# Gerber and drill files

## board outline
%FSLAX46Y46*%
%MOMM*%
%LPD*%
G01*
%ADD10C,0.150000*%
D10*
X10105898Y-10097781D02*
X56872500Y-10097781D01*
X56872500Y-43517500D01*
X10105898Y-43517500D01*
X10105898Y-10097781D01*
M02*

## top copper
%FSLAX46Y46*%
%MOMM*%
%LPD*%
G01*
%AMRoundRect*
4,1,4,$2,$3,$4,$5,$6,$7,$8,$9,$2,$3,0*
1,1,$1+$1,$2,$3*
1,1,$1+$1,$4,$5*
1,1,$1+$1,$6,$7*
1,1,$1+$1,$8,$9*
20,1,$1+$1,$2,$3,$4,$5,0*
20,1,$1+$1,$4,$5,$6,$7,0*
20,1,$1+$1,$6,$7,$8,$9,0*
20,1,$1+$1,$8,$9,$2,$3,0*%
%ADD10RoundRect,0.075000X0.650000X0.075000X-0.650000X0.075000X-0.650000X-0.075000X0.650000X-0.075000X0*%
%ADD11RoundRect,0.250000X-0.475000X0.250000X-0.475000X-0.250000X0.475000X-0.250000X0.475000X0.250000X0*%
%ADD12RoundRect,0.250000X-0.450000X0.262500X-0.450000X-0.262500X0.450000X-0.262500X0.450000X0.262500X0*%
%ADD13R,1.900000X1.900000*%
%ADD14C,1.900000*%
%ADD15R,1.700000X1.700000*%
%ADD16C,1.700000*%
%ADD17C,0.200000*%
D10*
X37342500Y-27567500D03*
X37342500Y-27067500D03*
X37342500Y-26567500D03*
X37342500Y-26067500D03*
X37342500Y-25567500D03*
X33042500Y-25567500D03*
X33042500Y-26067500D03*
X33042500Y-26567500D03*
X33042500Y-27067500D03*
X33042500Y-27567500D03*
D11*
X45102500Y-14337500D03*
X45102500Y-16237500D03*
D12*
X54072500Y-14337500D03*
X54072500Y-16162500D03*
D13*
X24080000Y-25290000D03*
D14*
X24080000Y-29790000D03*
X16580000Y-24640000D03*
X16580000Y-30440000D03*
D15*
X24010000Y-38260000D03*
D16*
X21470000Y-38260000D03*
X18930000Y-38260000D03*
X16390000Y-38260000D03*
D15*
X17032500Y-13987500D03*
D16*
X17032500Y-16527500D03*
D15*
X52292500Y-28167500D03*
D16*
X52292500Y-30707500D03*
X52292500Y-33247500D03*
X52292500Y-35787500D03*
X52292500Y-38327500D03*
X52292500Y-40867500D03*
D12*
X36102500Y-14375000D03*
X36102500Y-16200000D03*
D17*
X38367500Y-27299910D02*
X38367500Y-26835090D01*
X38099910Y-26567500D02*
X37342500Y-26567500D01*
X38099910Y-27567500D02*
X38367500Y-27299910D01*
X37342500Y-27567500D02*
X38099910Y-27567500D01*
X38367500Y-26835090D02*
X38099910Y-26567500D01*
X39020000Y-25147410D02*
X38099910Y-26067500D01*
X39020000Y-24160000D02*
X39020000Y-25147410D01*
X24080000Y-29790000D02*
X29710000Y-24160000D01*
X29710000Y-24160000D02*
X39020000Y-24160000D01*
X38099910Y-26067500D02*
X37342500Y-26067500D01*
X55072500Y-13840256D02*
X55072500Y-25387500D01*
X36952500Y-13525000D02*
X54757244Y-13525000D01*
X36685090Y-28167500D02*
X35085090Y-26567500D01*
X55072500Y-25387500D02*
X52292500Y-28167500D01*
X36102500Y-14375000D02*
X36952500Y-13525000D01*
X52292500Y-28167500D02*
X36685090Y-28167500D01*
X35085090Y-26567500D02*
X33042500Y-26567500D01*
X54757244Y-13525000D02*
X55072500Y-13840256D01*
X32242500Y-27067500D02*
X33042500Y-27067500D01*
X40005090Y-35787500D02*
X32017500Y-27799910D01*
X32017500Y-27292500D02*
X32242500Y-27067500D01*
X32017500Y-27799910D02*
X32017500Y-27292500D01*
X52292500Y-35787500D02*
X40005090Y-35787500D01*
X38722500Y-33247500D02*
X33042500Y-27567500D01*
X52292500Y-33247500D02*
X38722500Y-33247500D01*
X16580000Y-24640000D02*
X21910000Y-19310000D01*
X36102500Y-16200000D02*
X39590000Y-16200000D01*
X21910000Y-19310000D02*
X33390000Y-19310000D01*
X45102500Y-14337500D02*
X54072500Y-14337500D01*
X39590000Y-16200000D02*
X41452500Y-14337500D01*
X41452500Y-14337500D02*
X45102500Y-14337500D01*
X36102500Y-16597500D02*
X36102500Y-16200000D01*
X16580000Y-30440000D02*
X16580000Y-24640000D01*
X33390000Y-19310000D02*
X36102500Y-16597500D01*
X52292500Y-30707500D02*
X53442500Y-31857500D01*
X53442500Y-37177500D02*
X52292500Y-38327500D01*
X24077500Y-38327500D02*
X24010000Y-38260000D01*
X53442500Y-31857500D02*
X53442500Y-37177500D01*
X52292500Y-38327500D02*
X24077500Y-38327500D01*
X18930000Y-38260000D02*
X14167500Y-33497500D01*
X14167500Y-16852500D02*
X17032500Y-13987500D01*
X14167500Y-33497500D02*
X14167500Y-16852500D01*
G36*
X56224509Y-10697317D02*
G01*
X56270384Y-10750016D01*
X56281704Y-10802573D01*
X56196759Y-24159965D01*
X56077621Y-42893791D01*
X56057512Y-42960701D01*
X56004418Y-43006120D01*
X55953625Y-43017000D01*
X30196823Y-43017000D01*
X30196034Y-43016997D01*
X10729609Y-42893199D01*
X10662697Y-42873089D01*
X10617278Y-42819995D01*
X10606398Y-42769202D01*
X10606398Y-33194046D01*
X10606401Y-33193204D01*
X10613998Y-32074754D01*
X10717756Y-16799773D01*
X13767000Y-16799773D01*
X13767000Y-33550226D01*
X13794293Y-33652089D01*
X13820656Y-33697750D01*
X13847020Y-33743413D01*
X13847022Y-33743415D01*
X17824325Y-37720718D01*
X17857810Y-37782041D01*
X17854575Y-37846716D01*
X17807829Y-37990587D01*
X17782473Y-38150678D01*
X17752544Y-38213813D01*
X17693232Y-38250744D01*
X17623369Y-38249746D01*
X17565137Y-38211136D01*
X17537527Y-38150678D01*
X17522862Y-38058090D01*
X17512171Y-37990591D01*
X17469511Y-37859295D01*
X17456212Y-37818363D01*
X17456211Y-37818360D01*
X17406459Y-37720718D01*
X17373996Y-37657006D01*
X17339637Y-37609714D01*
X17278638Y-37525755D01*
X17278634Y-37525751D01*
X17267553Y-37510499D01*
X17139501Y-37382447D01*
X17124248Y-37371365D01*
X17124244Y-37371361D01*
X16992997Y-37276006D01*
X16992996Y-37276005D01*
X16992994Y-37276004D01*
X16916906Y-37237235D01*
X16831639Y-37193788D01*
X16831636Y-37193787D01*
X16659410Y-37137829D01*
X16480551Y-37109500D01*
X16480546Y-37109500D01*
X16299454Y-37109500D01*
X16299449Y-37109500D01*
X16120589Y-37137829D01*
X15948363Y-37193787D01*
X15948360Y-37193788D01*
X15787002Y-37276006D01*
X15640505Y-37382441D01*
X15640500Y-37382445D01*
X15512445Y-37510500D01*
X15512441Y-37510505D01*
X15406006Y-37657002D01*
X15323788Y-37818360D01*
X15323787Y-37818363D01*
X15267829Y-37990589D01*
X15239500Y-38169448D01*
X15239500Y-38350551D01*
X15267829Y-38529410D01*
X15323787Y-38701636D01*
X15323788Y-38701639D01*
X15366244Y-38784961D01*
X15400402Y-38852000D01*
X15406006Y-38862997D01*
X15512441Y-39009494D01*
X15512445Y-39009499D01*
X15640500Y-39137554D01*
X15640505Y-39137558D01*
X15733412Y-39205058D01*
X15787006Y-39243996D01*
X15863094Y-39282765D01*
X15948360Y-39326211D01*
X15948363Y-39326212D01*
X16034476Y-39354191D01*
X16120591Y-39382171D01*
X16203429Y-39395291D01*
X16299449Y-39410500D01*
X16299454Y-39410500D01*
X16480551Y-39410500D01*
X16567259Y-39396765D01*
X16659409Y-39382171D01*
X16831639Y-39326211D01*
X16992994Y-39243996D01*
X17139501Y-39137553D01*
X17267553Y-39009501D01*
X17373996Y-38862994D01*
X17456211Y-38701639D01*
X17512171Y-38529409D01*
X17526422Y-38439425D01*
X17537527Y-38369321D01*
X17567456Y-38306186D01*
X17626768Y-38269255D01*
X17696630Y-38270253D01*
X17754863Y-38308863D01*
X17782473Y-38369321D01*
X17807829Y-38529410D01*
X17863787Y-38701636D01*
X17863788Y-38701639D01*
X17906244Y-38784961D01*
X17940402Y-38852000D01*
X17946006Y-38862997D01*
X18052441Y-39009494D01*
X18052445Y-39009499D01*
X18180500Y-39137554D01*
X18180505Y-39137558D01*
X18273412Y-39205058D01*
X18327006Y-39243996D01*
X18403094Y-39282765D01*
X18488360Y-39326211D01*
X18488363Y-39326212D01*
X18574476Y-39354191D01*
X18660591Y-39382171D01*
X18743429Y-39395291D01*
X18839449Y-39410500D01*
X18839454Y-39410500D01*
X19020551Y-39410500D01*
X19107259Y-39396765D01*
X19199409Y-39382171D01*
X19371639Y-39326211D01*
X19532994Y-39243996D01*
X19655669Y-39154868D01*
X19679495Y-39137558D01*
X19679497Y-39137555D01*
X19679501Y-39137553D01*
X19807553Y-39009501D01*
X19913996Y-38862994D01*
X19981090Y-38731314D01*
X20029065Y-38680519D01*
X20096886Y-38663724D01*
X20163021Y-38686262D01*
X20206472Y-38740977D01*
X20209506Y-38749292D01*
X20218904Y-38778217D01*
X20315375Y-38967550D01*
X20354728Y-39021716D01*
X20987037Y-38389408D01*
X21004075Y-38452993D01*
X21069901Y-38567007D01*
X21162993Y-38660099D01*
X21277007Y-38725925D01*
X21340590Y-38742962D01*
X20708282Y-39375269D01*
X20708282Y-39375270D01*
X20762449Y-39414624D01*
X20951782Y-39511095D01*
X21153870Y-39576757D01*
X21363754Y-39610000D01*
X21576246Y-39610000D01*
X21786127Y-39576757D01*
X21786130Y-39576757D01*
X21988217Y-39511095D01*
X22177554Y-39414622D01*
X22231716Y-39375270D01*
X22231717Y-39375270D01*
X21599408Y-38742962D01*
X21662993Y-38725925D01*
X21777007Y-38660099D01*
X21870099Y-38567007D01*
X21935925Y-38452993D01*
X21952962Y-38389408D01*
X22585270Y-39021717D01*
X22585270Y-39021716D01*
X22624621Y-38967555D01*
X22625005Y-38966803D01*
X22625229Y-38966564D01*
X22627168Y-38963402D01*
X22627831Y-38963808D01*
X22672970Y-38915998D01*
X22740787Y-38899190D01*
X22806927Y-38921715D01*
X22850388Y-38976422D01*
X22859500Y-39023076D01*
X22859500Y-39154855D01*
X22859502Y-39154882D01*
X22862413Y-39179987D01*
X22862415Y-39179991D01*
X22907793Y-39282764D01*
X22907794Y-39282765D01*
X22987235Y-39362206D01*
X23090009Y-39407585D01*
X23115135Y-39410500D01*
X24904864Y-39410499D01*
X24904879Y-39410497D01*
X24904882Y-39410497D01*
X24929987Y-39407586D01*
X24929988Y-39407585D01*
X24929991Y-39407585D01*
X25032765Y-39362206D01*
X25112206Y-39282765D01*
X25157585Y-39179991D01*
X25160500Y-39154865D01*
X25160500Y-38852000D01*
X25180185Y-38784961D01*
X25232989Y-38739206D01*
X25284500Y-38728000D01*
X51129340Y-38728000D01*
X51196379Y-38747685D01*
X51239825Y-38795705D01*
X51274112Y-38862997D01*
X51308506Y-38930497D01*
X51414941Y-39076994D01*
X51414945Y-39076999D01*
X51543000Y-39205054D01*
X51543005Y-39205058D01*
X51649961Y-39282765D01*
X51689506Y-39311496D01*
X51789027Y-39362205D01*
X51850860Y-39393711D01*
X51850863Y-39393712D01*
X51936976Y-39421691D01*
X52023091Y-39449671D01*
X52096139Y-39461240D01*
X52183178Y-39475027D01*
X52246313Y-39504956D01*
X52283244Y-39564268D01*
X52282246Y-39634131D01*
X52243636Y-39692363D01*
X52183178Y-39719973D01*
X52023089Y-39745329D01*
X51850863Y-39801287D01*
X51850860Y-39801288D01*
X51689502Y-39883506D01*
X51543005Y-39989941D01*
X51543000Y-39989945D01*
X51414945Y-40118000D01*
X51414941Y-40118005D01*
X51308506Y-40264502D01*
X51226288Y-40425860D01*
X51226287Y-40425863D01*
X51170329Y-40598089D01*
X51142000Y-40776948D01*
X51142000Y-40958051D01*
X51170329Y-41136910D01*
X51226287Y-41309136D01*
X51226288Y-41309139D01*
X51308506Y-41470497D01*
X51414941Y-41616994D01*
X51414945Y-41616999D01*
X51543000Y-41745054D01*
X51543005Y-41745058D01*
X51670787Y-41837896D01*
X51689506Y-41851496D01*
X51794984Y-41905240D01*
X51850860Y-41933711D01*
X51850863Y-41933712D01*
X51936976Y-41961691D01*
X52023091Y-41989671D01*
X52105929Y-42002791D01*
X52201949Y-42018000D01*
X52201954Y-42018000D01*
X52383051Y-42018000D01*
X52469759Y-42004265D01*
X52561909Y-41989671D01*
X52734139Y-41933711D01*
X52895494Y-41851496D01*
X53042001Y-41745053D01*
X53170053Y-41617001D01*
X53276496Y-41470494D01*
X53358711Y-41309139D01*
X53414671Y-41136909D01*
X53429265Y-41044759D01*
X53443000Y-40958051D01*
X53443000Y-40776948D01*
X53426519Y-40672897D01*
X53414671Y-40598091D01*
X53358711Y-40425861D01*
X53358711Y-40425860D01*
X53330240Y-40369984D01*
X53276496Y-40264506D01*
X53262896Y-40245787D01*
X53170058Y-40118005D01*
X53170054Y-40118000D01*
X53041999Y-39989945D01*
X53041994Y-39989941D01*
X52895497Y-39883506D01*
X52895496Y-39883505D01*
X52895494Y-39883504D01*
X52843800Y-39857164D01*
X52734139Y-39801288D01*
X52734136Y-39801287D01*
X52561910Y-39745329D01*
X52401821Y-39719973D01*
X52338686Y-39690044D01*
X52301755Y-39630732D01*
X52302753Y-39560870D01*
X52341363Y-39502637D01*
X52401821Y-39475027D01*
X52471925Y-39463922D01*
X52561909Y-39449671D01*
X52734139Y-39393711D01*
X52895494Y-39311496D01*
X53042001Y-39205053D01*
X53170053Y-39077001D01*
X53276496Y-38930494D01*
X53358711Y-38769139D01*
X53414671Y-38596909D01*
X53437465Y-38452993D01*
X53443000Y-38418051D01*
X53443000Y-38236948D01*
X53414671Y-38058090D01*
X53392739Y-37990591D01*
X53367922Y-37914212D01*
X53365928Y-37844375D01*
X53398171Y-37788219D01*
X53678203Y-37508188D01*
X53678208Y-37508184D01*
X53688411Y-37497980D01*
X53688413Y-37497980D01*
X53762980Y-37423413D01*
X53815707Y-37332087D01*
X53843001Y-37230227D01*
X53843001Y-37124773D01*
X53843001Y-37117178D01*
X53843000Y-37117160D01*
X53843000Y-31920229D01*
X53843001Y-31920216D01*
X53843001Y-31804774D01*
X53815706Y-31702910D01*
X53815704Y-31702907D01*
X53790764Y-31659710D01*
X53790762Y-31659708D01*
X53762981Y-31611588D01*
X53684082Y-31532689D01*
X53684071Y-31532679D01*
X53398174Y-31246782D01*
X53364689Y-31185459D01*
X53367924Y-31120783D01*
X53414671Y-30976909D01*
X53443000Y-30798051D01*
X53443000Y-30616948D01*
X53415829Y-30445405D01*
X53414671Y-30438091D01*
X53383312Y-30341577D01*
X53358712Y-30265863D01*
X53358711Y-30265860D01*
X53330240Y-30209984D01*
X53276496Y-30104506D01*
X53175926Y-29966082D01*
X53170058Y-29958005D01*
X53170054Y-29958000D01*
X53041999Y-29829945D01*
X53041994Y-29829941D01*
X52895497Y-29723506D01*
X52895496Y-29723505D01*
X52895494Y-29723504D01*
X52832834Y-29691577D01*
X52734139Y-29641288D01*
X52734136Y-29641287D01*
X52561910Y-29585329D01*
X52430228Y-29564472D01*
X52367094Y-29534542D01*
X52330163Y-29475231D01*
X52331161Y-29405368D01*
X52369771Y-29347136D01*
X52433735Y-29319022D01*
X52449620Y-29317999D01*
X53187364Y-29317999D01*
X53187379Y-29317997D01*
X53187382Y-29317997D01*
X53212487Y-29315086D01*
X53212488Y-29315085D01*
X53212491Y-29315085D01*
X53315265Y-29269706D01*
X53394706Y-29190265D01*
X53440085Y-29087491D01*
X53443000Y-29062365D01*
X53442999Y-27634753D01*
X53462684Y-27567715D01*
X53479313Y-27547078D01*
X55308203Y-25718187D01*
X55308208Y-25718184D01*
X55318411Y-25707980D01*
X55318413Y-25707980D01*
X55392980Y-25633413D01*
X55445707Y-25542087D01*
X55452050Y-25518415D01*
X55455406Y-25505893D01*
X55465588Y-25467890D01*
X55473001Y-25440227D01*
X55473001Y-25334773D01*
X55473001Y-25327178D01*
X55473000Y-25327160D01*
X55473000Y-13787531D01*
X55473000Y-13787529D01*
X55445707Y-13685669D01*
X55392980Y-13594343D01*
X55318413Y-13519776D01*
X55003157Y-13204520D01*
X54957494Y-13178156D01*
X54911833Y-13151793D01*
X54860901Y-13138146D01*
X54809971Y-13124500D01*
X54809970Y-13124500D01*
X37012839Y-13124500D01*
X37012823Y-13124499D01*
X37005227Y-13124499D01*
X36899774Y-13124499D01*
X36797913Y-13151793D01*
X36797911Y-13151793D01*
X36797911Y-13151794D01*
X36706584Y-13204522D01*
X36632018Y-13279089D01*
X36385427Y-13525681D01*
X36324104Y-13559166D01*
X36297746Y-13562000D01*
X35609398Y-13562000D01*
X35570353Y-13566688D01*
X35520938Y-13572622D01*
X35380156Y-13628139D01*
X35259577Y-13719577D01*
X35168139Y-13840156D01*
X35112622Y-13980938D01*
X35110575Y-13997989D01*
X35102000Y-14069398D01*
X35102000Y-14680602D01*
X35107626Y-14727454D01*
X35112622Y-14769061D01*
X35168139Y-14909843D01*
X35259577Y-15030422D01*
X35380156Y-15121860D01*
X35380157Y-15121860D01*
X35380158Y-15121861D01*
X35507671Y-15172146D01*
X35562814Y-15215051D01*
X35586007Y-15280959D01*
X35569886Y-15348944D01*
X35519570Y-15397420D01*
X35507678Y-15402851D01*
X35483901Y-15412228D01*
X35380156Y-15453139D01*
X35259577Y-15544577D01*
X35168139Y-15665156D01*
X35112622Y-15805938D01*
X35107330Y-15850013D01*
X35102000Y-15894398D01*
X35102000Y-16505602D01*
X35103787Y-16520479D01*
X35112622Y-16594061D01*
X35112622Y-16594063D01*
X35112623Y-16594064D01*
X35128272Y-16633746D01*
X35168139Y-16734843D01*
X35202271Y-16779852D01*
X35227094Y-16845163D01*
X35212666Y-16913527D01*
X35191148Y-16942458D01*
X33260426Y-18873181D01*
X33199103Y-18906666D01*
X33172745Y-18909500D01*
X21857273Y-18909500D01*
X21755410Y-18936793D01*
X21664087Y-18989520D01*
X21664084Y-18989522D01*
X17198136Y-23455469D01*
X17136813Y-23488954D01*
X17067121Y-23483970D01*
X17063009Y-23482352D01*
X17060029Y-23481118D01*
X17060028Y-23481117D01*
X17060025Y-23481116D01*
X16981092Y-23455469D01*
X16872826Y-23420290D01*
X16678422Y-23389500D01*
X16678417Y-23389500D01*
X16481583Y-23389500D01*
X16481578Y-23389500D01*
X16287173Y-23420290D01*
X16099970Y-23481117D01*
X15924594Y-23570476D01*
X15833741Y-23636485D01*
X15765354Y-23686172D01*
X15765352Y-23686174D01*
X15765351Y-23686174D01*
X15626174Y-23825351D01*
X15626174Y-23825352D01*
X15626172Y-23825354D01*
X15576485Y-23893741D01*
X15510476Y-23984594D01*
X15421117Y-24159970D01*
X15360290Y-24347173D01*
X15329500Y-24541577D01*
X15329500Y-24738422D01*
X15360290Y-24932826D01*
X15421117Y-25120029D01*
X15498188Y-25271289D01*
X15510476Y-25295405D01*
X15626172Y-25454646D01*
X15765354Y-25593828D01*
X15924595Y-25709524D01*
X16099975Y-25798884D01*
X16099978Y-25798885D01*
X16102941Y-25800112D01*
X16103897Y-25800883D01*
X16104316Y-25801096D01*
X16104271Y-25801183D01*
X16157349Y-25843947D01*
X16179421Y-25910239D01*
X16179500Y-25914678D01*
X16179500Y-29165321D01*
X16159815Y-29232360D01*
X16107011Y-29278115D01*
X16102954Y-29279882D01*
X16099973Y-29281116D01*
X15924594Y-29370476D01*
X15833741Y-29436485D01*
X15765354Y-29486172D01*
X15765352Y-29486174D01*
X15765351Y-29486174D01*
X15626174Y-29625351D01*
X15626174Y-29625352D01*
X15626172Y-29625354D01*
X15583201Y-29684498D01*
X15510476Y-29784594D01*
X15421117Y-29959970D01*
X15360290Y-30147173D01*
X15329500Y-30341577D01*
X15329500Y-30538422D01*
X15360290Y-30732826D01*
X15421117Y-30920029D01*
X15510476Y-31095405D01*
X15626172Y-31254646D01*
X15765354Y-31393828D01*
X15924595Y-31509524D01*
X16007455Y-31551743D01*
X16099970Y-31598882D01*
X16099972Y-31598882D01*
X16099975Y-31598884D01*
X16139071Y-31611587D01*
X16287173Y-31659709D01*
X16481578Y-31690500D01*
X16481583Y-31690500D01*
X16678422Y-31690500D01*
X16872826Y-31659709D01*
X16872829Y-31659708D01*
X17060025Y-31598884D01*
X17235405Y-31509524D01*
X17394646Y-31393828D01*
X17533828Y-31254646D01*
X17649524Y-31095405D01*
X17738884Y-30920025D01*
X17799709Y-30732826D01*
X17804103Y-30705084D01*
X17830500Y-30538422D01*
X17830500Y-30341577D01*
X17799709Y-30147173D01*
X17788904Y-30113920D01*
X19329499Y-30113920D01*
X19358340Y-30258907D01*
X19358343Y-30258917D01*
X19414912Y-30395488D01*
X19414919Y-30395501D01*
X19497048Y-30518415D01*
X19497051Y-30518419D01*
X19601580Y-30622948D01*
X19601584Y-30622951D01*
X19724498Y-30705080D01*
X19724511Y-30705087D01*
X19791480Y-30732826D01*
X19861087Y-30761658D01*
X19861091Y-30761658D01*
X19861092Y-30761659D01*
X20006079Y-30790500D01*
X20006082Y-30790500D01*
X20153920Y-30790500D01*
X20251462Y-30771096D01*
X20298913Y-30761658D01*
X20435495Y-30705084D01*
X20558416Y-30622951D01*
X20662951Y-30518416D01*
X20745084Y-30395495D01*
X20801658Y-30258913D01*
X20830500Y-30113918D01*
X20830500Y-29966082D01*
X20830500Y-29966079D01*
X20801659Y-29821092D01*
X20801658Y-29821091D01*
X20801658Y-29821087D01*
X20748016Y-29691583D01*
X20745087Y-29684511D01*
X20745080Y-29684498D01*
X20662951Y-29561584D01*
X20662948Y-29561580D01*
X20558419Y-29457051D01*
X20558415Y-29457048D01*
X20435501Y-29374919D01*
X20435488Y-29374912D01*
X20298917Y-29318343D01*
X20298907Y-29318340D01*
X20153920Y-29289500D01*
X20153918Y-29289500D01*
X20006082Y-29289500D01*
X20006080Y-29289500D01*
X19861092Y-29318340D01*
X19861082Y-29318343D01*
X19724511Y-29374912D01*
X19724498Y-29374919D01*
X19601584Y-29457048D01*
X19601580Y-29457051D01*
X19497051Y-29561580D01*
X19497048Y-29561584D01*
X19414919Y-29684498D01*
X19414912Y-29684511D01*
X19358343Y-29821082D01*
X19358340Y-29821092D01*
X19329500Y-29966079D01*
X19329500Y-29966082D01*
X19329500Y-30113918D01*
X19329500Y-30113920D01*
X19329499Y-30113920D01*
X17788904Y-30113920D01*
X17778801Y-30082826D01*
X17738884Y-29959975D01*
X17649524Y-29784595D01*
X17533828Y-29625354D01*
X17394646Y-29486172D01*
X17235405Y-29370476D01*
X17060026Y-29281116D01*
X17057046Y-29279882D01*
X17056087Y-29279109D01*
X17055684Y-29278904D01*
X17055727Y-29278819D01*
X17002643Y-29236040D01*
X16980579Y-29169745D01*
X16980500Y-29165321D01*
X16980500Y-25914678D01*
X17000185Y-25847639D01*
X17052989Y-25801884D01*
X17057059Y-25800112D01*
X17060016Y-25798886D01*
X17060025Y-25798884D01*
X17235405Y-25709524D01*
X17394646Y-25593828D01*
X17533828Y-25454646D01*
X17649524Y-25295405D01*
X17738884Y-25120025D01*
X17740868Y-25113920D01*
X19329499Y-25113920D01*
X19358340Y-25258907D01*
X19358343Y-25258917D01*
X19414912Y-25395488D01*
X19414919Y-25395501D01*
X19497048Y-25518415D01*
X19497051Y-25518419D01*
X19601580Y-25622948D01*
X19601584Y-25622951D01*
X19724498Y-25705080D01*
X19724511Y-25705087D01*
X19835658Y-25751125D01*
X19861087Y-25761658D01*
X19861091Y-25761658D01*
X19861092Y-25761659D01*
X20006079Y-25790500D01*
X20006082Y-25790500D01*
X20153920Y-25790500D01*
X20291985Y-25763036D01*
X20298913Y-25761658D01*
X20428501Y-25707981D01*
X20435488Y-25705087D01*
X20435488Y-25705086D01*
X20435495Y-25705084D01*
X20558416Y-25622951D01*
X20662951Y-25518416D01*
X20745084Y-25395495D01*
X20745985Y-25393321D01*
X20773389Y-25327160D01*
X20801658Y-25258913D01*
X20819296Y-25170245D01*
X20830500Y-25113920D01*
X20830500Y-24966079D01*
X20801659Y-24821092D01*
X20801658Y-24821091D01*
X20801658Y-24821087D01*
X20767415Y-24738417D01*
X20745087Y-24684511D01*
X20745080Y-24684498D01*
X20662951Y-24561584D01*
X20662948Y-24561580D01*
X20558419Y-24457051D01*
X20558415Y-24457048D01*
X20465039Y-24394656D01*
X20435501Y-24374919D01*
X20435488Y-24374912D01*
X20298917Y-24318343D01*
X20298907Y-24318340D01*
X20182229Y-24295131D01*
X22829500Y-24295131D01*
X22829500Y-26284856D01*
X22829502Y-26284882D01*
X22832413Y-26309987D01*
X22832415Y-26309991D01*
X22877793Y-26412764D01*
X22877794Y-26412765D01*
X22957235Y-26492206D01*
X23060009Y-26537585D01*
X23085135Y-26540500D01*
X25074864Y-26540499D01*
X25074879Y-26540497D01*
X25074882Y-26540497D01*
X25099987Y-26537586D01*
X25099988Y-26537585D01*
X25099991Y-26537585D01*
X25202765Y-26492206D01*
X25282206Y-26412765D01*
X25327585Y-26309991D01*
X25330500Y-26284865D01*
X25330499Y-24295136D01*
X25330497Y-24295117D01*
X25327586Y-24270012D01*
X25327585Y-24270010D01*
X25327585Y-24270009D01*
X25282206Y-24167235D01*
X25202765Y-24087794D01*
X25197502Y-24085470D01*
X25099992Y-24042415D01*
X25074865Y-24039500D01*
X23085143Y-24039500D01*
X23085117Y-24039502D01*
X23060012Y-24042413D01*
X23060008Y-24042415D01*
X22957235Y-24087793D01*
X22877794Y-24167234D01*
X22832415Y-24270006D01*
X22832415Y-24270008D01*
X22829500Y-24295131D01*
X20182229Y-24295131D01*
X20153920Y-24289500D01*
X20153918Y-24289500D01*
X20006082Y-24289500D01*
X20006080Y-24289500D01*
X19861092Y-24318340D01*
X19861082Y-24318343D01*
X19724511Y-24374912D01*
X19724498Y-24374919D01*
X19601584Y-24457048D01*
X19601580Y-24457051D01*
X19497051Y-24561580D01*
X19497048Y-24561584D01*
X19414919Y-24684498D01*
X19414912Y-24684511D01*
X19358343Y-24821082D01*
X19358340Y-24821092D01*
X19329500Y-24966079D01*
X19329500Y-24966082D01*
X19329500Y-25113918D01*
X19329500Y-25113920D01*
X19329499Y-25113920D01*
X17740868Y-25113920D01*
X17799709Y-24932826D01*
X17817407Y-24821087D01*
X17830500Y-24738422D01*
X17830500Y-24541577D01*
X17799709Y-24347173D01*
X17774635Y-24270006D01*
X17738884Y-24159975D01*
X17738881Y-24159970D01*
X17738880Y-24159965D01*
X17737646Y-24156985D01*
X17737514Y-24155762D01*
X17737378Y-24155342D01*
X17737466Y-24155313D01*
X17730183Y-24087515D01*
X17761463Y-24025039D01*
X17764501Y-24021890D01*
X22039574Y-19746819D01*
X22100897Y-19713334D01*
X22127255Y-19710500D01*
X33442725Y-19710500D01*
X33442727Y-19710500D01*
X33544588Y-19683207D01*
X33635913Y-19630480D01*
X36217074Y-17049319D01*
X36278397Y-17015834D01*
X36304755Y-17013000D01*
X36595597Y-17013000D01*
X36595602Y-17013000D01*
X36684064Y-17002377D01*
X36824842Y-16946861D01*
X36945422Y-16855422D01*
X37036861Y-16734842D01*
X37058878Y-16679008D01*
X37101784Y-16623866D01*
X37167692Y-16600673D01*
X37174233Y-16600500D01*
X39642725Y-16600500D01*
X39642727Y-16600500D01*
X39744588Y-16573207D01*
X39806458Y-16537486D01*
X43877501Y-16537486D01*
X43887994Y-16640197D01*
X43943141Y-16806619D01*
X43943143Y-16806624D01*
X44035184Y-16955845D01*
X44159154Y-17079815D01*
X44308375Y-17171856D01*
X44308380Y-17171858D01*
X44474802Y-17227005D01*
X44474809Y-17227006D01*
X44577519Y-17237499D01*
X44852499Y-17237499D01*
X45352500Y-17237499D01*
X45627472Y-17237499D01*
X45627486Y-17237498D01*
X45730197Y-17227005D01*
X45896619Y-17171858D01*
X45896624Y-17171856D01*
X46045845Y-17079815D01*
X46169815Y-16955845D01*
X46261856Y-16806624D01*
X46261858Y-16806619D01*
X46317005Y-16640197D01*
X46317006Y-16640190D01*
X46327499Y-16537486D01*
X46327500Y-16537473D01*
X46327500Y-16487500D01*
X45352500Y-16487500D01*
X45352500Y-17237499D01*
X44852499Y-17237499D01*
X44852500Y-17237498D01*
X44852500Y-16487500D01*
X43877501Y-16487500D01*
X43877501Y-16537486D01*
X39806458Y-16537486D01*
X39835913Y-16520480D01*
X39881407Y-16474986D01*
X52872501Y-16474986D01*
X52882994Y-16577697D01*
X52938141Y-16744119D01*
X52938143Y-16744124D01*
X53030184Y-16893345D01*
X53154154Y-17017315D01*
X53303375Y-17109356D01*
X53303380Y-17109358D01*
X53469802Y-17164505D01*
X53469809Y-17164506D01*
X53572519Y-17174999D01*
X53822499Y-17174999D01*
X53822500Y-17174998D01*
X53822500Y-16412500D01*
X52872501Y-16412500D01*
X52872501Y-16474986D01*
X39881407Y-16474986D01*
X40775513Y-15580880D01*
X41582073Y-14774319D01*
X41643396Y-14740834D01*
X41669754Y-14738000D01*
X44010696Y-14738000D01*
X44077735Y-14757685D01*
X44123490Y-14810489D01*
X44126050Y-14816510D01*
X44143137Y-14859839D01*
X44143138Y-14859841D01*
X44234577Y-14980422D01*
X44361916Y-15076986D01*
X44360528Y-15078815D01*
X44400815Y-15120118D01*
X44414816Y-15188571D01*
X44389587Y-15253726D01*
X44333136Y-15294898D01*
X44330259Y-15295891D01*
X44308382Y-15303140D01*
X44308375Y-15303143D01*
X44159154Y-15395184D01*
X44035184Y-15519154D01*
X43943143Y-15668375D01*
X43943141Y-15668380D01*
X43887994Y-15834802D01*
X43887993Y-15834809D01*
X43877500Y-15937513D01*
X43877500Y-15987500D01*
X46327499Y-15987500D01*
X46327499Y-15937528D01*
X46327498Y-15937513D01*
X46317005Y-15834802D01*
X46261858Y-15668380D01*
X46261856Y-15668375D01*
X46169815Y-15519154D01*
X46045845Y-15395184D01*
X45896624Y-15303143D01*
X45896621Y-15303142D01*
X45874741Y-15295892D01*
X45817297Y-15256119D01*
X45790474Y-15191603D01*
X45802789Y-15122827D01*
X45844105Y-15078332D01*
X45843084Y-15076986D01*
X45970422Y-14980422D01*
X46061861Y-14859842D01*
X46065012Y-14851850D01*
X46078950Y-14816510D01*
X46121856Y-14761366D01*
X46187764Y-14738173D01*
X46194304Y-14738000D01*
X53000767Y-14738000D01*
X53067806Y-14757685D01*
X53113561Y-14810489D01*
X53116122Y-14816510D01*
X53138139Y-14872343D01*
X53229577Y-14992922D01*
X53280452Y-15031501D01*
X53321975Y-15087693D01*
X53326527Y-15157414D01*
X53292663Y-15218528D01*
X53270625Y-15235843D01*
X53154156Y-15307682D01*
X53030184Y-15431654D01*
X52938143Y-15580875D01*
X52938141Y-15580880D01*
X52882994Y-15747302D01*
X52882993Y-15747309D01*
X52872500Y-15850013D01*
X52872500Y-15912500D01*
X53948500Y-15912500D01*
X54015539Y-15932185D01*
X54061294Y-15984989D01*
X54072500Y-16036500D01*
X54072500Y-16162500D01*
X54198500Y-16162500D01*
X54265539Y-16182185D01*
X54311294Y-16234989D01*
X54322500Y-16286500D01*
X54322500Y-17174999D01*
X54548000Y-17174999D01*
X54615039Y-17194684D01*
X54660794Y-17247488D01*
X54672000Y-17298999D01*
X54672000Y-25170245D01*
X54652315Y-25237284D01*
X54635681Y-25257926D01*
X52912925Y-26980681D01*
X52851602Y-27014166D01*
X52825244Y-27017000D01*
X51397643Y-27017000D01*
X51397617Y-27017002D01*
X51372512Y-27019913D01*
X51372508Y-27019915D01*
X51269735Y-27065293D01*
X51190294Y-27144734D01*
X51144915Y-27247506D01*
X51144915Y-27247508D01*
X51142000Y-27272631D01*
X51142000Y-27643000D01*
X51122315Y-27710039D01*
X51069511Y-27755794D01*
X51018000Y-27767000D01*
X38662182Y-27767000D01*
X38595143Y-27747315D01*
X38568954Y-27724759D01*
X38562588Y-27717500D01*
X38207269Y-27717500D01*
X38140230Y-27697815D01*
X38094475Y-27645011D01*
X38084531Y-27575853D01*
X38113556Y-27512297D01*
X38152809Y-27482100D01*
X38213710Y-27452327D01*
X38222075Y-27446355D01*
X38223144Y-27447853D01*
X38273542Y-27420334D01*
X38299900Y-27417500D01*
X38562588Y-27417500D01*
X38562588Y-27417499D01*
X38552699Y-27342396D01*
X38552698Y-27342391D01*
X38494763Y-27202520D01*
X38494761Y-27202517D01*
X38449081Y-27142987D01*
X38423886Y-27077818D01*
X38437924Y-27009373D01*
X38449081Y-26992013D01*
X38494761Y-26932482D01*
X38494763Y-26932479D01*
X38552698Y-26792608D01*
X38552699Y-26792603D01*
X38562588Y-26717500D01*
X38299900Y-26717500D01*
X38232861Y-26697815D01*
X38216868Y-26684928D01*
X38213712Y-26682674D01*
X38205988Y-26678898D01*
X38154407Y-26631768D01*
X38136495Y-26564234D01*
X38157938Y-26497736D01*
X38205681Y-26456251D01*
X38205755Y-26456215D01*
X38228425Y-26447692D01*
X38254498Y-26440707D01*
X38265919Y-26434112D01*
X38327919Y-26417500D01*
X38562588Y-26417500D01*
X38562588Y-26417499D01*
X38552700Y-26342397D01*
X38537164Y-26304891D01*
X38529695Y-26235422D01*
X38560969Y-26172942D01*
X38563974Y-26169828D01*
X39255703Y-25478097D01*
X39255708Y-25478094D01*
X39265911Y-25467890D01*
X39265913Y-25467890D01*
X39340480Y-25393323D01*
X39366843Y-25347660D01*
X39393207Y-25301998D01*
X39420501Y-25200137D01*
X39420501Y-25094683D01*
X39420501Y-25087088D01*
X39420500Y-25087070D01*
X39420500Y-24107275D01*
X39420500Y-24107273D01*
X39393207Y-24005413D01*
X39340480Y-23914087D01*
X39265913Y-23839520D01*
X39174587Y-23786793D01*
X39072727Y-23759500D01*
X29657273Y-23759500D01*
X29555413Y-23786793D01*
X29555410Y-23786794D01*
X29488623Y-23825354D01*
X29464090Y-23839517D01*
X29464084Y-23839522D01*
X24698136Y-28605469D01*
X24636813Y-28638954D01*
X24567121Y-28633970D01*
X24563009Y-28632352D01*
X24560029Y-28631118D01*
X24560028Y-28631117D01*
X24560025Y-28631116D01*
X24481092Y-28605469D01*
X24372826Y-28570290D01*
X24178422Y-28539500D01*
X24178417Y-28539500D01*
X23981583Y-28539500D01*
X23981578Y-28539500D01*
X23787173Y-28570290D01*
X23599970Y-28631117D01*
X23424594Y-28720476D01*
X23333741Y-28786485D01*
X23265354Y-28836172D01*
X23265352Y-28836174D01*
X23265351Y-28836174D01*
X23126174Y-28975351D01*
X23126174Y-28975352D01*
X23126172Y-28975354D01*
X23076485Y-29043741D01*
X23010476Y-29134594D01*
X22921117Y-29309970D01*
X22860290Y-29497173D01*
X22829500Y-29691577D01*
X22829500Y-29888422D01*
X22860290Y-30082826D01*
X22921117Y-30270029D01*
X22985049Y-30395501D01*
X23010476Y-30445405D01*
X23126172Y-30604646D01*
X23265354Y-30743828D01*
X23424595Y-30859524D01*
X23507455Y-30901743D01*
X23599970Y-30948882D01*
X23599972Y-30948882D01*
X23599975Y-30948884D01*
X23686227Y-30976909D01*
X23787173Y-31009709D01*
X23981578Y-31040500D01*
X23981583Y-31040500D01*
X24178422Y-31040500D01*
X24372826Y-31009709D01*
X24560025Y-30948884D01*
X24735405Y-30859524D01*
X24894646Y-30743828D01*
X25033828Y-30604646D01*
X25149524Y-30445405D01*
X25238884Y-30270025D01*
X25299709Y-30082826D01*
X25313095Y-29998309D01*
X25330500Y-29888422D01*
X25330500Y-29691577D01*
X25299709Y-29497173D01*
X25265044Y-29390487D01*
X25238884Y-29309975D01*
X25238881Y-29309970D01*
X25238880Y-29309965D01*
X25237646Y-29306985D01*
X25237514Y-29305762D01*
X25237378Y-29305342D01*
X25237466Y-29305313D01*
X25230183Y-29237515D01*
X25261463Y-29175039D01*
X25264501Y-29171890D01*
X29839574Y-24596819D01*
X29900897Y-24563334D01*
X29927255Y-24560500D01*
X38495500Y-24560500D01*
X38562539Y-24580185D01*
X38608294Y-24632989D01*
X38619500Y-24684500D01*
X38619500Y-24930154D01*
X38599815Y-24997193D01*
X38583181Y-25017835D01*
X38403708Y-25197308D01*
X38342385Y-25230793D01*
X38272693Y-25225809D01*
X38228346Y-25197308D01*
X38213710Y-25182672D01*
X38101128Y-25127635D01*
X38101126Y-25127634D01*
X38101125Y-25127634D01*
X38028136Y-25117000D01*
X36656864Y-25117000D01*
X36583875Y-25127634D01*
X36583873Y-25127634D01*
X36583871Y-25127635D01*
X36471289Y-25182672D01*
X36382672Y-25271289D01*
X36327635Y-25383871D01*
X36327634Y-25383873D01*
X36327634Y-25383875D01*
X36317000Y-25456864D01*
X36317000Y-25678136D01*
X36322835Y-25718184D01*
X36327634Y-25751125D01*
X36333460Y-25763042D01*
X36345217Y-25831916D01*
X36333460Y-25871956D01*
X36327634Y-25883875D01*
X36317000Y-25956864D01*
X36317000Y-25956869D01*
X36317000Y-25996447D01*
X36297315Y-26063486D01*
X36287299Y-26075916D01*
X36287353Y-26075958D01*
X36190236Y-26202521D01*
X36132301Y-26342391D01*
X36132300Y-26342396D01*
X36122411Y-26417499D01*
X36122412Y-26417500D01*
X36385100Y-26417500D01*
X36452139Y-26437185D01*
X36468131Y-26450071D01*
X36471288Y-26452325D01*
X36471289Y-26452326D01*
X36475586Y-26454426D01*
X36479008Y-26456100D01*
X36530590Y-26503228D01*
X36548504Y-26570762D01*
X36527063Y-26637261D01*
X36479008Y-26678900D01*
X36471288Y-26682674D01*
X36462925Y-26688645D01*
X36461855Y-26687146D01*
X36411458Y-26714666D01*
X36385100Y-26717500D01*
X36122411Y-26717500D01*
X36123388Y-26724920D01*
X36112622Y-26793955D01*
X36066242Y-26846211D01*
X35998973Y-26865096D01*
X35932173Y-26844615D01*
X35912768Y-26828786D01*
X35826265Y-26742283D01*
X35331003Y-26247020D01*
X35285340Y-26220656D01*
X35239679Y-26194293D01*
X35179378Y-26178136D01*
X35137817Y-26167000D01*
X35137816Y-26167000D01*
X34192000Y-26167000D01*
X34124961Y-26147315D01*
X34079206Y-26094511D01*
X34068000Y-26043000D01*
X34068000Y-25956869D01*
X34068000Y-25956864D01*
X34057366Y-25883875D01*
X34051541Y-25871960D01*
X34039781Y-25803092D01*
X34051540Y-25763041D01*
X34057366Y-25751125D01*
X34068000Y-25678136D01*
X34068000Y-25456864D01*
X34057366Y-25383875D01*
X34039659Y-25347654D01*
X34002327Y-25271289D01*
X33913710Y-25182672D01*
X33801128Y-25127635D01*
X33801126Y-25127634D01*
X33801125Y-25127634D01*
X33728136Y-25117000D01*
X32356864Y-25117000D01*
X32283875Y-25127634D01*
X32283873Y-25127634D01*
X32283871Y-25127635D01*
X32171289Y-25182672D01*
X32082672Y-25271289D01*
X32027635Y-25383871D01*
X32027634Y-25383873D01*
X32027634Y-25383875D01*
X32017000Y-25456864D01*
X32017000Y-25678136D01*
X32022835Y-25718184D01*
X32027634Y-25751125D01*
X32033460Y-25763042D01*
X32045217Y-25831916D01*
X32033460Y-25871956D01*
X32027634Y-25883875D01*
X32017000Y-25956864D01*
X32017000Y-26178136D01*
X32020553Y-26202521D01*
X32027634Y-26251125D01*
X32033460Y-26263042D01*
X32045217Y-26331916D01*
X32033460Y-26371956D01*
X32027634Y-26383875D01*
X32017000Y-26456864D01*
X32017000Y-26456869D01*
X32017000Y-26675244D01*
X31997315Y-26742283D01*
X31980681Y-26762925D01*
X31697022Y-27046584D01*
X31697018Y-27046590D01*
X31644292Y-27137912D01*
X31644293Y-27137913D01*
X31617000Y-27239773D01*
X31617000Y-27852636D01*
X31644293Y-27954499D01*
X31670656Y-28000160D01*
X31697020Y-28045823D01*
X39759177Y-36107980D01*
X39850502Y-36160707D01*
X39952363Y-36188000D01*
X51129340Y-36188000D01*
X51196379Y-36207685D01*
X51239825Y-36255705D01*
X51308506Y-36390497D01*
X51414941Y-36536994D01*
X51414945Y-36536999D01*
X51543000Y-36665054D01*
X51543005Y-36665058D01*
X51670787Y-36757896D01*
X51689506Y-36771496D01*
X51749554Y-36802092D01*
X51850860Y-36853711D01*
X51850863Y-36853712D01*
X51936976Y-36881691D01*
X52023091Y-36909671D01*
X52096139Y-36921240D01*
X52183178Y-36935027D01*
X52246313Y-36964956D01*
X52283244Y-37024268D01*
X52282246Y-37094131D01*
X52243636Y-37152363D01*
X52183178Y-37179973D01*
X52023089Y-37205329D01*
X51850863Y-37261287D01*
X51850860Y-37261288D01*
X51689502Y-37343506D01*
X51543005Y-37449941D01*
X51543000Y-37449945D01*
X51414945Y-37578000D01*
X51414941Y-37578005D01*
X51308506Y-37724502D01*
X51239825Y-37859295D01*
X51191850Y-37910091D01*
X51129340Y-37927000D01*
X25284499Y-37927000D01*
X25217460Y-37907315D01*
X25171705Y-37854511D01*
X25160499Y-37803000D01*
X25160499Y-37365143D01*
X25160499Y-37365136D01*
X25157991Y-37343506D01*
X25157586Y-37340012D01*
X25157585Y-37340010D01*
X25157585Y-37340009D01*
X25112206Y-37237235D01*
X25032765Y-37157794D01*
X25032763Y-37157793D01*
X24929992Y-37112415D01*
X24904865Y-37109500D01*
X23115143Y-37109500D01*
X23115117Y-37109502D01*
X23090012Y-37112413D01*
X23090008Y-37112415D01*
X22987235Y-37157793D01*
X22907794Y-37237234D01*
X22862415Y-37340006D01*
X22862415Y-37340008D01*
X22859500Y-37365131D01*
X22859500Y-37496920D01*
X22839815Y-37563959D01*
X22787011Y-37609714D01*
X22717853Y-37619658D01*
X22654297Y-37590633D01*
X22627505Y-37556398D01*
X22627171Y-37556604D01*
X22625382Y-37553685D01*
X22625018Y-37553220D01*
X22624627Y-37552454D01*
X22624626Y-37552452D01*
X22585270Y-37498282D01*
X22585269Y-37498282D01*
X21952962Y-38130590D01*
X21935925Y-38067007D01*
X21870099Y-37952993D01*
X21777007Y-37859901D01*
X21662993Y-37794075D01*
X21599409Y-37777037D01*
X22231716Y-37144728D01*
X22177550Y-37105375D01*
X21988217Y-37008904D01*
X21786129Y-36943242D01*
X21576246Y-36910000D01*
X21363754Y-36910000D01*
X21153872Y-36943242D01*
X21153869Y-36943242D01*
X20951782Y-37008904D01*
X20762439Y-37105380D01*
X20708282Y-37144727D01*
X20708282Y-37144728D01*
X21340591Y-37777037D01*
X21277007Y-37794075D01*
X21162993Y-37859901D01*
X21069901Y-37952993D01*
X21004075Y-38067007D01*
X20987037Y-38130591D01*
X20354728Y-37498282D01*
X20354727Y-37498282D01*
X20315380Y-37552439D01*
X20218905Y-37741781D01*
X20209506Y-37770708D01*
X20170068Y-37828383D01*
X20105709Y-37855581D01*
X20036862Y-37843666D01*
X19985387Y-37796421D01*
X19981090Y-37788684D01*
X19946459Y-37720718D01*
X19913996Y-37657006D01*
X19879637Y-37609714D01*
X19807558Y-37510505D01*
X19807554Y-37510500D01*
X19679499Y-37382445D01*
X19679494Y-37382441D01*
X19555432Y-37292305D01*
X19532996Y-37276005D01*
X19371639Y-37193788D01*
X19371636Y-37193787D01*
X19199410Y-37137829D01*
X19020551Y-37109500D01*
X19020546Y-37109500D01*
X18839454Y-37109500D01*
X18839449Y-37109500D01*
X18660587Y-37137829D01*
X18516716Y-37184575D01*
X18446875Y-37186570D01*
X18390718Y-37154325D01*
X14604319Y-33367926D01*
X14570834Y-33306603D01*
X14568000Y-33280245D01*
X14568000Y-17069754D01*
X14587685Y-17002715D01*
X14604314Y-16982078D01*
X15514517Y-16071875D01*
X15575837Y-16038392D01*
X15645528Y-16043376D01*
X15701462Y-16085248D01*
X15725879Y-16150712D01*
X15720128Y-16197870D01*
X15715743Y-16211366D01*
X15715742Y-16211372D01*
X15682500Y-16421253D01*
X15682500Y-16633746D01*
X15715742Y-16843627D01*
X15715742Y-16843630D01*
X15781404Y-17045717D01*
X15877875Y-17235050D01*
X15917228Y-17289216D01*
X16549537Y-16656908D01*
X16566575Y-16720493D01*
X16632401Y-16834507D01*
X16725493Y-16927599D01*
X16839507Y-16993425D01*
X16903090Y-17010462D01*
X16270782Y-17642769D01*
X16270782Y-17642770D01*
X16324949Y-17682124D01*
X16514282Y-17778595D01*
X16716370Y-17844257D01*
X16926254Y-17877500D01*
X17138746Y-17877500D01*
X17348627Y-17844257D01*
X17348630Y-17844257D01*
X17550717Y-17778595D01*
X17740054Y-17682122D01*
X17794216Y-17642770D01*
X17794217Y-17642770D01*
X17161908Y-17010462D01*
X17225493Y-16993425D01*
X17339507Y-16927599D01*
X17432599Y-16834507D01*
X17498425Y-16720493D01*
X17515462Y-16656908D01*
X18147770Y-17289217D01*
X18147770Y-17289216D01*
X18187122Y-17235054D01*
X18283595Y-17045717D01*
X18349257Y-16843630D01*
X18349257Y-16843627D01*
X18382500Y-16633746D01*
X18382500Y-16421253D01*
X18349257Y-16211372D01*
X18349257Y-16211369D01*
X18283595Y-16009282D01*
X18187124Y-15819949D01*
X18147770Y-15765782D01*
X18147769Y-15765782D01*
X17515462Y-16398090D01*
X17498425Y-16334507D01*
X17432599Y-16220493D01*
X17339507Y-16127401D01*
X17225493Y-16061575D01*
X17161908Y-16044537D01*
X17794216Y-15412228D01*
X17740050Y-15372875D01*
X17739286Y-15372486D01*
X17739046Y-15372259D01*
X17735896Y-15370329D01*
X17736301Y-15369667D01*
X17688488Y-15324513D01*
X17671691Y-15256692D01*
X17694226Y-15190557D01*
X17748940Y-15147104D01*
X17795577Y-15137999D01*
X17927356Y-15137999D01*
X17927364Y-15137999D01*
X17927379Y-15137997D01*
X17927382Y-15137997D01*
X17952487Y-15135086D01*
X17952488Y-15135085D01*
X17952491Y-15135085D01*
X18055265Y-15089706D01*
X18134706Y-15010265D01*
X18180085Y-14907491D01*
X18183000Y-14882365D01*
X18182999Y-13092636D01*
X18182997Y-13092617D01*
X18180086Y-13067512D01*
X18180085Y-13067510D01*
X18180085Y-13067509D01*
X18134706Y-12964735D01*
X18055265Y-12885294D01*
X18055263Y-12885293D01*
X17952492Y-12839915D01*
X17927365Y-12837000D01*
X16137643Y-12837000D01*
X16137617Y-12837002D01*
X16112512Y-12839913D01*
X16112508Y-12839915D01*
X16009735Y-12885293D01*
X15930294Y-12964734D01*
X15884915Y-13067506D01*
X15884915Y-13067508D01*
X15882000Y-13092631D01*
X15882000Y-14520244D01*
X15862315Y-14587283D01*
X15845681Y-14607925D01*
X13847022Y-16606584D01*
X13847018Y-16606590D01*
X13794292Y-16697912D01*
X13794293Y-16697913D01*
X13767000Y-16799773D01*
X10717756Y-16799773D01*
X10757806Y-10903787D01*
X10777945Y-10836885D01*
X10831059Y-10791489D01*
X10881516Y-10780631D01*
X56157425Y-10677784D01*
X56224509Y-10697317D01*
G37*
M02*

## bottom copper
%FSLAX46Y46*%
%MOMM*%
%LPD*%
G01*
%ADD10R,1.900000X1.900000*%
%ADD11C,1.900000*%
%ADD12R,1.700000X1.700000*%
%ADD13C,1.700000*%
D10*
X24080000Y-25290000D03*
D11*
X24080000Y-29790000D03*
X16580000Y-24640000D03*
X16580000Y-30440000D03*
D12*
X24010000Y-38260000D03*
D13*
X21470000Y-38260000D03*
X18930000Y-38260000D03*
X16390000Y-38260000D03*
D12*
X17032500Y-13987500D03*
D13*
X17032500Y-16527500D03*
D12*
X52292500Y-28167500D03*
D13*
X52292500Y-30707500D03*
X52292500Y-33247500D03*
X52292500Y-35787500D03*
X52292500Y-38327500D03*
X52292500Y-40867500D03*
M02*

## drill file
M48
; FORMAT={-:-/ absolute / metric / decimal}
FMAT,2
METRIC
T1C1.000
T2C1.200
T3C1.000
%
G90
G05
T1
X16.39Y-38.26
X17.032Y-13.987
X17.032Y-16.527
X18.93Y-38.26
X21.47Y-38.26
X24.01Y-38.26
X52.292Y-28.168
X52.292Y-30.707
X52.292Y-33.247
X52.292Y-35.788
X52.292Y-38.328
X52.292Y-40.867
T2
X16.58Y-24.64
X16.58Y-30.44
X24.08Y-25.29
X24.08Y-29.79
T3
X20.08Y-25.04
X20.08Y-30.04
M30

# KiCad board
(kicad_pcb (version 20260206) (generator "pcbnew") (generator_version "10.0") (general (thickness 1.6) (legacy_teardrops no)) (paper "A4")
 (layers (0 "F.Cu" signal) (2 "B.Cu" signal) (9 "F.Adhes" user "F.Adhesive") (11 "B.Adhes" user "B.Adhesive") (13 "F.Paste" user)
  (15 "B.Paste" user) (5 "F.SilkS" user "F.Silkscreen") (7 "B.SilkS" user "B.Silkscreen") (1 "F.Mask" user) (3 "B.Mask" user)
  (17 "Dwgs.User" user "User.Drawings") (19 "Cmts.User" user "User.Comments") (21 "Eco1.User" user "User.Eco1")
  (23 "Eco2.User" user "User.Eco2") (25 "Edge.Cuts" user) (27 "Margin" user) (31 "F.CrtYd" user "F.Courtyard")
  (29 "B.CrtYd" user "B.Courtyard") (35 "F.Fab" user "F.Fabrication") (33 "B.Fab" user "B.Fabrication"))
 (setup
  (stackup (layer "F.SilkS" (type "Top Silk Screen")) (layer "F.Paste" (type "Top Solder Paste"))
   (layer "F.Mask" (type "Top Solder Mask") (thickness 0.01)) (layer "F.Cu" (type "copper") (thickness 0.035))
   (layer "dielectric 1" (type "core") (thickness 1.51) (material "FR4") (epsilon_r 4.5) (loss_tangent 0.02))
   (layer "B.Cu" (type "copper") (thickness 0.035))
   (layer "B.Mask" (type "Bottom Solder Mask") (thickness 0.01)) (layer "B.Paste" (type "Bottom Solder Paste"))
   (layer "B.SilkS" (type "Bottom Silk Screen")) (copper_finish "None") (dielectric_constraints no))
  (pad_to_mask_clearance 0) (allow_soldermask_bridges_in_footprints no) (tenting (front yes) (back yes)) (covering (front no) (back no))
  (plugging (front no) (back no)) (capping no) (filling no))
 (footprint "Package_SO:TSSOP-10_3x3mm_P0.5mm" (layer "F.Cu") (at 35.1925 26.5675 180)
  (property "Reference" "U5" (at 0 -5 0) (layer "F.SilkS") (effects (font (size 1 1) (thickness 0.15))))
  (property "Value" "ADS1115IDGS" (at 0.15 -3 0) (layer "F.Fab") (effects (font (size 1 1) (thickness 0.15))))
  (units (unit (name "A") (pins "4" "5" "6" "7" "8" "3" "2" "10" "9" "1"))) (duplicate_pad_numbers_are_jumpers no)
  (pad "1" smd roundrect (at -2.15 -1 180) (size 1.45 0.3) (layers "F.Cu" "F.Mask" "F.Paste") (roundrect_rratio 0.25) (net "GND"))
  (pad "2" smd roundrect (at -2.15 -0.5 180) (size 1.45 0.3) (layers "F.Cu" "F.Mask" "F.Paste") (roundrect_rratio 0.25)
   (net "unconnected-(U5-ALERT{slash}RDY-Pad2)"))
  (pad "3" smd roundrect (at -2.15 0 180) (size 1.45 0.3) (layers "F.Cu" "F.Mask" "F.Paste") (roundrect_rratio 0.25) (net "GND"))
  (pad "4" smd roundrect (at -2.15 0.5 180) (size 1.45 0.3) (layers "F.Cu" "F.Mask" "F.Paste") (roundrect_rratio 0.25) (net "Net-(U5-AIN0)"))
  (pad "5" smd roundrect (at -2.15 1 180) (size 1.45 0.3) (layers "F.Cu" "F.Mask" "F.Paste") (roundrect_rratio 0.25)
   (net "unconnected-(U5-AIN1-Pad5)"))
  (pad "6" smd roundrect (at 2.15 1 180) (size 1.45 0.3) (layers "F.Cu" "F.Mask" "F.Paste") (roundrect_rratio 0.25)
   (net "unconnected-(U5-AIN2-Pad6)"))
  (pad "7" smd roundrect (at 2.15 0.5 180) (size 1.45 0.3) (layers "F.Cu" "F.Mask" "F.Paste") (roundrect_rratio 0.25)
   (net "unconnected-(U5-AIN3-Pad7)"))
  (pad "8" smd roundrect (at 2.15 0 180) (size 1.45 0.3) (layers "F.Cu" "F.Mask" "F.Paste") (roundrect_rratio 0.25) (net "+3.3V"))
  (pad "9" smd roundrect (at 2.15 -0.5 180) (size 1.45 0.3) (layers "F.Cu" "F.Mask" "F.Paste") (roundrect_rratio 0.25)
   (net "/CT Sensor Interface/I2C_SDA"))
  (pad "10" smd roundrect (at 2.15 -1 180) (size 1.45 0.3) (layers "F.Cu" "F.Mask" "F.Paste") (roundrect_rratio 0.25)
   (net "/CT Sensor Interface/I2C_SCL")))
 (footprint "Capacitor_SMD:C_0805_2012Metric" (layer "F.Cu") (at 45.1025 15.2875 -90)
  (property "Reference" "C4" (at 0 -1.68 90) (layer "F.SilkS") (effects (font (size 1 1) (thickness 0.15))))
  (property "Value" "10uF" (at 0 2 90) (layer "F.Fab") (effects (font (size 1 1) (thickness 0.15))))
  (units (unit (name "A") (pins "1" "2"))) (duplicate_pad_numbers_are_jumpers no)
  (pad "1" smd roundrect (at -0.95 0 270) (size 1 1.45) (layers "F.Cu" "F.Mask" "F.Paste") (roundrect_rratio 0.25) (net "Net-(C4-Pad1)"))
  (pad "2" smd roundrect (at 0.95 0 270) (size 1 1.45) (layers "F.Cu" "F.Mask" "F.Paste") (roundrect_rratio 0.25) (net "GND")))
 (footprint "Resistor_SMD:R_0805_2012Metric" (layer "F.Cu") (at 54.0725 15.25 -90)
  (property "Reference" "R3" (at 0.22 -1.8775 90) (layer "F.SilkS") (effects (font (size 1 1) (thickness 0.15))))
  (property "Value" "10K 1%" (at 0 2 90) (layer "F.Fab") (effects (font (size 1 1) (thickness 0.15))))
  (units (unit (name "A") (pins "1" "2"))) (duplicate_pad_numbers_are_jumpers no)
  (pad "1" smd roundrect (at -0.9125 0 270) (size 1.025 1.4) (layers "F.Cu" "F.Mask" "F.Paste") (roundrect_rratio 0.243902)
   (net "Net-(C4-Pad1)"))
  (pad "2" smd roundrect (at 0.9125 0 270) (size 1.025 1.4) (layers "F.Cu" "F.Mask" "F.Paste") (roundrect_rratio 0.243902) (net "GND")))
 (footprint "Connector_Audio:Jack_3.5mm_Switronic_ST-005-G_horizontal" (layer "F.Cu") (at 17.58 27.54)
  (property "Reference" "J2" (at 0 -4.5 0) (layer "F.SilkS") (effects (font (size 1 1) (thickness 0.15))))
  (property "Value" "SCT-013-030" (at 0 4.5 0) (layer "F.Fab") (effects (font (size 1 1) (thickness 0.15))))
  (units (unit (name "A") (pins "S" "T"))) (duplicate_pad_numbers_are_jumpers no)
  (pad "" np_thru_hole circle (at 2.5 -2.5) (size 1 1) (drill 1) (layers "*.Cu" "*.Mask"))
  (pad "" np_thru_hole circle (at 2.5 2.5) (size 1 1) (drill 1) (layers "*.Cu" "*.Mask"))
  (pad "R" thru_hole rect (at 6.5 -2.25) (size 1.9 1.9) (drill 1.2) (layers "*.Cu" "*.Mask") (remove_unused_layers no))
  (pad "S" thru_hole circle (at 6.5 2.25) (size 1.9 1.9) (drill 1.2) (layers "*.Cu" "*.Mask") (remove_unused_layers no)
   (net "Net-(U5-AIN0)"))
  (pad "T" thru_hole circle (at -1 -2.9) (size 1.9 1.9) (drill 1.2) (layers "*.Cu" "*.Mask") (remove_unused_layers no) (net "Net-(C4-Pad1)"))
  (pad "T" thru_hole circle (at -1 2.9) (size 1.9 1.9) (drill 1.2) (layers "*.Cu" "*.Mask") (remove_unused_layers no) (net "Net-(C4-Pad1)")))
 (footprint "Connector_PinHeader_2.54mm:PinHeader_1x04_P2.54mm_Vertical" (layer "F.Cu") (at 24.01 38.26 -90)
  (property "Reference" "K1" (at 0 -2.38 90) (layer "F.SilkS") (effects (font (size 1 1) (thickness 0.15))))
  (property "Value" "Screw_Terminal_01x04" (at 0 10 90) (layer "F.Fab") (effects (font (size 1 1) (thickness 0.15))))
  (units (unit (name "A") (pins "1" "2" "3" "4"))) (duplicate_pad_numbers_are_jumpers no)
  (pad "1" thru_hole rect (at 0 0 270) (size 1.7 1.7) (drill 1) (layers "*.Cu" "*.Mask") (remove_unused_layers no)
   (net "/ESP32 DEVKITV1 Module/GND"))
  (pad "2" thru_hole circle (at 0 2.54 270) (size 1.7 1.7) (drill 1) (layers "*.Cu" "*.Mask") (remove_unused_layers no) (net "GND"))
  (pad "3" thru_hole circle (at 0 5.08 270) (size 1.7 1.7) (drill 1) (layers "*.Cu" "*.Mask") (remove_unused_layers no) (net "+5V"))
  (pad "4" thru_hole circle (at 0 7.62 270) (size 1.7 1.7) (drill 1) (layers "*.Cu" "*.Mask") (remove_unused_layers no)
   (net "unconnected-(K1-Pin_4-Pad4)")))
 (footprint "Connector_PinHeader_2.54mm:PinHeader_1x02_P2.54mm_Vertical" (layer "F.Cu") (at 17.0325 13.9875)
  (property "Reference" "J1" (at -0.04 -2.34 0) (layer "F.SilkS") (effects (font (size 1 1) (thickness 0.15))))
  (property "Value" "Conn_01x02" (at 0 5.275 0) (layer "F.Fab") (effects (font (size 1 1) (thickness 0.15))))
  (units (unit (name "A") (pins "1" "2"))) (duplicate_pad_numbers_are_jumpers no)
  (pad "1" thru_hole rect (at 0 0) (size 1.7 1.7) (drill 1) (layers "*.Cu" "*.Mask") (remove_unused_layers no) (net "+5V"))
  (pad "2" thru_hole circle (at 0 2.54) (size 1.7 1.7) (drill 1) (layers "*.Cu" "*.Mask") (remove_unused_layers no) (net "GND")))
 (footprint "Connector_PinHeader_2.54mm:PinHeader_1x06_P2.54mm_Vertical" (layer "F.Cu") (at 52.2925 28.1675)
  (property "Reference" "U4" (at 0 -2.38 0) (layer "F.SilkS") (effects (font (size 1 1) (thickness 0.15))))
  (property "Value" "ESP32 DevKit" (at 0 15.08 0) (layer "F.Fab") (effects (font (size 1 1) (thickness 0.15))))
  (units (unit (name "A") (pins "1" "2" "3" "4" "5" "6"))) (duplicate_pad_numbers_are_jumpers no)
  (pad "1" thru_hole rect (at 0 0) (size 1.7 1.7) (drill 1) (layers "*.Cu" "*.Mask") (remove_unused_layers no) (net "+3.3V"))
  (pad "2" thru_hole circle (at 0 2.54) (size 1.7 1.7) (drill 1) (layers "*.Cu" "*.Mask") (remove_unused_layers no)
   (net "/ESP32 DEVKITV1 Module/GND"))
  (pad "3" thru_hole circle (at 0 5.08) (size 1.7 1.7) (drill 1) (layers "*.Cu" "*.Mask") (remove_unused_layers no)
   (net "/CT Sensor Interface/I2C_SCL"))
  (pad "4" thru_hole circle (at 0 7.62) (size 1.7 1.7) (drill 1) (layers "*.Cu" "*.Mask") (remove_unused_layers no)
   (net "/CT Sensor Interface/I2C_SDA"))
  (pad "5" thru_hole circle (at 0 10.16) (size 1.7 1.7) (drill 1) (layers "*.Cu" "*.Mask") (remove_unused_layers no)
   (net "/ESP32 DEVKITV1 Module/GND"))
  (pad "6" thru_hole circle (at 0 12.7) (size 1.7 1.7) (drill 1) (layers "*.Cu" "*.Mask") (remove_unused_layers no)
   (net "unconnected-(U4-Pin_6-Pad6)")))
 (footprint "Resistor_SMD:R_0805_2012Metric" (layer "F.Cu") (at 36.1025 15.2875 -90)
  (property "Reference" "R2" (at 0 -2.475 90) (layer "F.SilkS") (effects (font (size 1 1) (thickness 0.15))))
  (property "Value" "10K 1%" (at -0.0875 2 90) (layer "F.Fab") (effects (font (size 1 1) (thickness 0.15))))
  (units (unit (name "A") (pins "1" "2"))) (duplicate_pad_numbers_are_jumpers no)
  (pad "1" smd roundrect (at -0.9125 0 270) (size 1.025 1.4) (layers "F.Cu" "F.Mask" "F.Paste") (roundrect_rratio 0.243902) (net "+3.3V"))
  (pad "2" smd roundrect (at 0.9125 0 270) (size 1.025 1.4) (layers "F.Cu" "F.Mask" "F.Paste") (roundrect_rratio 0.243902)
   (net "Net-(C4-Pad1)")))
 (gr_rect (start 10.105898 10.097781) (end 56.8725 43.5175) (stroke (width 0.15) (type solid)) (fill no) (layer "Edge.Cuts"))
 (segment (start 38.3675 27.29991) (end 38.3675 26.83509) (width 0.2) (layer "F.Cu") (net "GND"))
 (segment (start 38.09991 26.5675) (end 37.3425 26.5675) (width 0.2) (layer "F.Cu") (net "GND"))
 (segment (start 38.09991 27.5675) (end 38.3675 27.29991) (width 0.2) (layer "F.Cu") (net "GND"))
 (segment (start 37.3425 27.5675) (end 38.09991 27.5675) (width 0.2) (layer "F.Cu") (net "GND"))
 (segment (start 38.3675 26.83509) (end 38.09991 26.5675) (width 0.2) (layer "F.Cu") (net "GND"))
 (segment (start 39.02 25.14741) (end 38.09991 26.0675) (width 0.2) (layer "F.Cu") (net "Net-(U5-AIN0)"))
 (segment (start 39.02 24.16) (end 39.02 25.14741) (width 0.2) (layer "F.Cu") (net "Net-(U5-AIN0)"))
 (segment (start 24.08 29.79) (end 29.71 24.16) (width 0.2) (layer "F.Cu") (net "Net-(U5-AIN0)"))
 (segment (start 29.71 24.16) (end 39.02 24.16) (width 0.2) (layer "F.Cu") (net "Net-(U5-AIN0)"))
 (segment (start 38.09991 26.0675) (end 37.3425 26.0675) (width 0.2) (layer "F.Cu") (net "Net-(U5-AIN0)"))
 (segment (start 55.0725 13.840256) (end 55.0725 25.3875) (width 0.2) (layer "F.Cu") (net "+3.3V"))
 (segment (start 36.9525 13.525) (end 54.757244 13.525) (width 0.2) (layer "F.Cu") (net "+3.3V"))
 (segment (start 36.68509 28.1675) (end 35.08509 26.5675) (width 0.2) (layer "F.Cu") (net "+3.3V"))
 (segment (start 55.0725 25.3875) (end 52.2925 28.1675) (width 0.2) (layer "F.Cu") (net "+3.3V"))
 (segment (start 36.1025 14.375) (end 36.9525 13.525) (width 0.2) (layer "F.Cu") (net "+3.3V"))
 (segment (start 52.2925 28.1675) (end 36.68509 28.1675) (width 0.2) (layer "F.Cu") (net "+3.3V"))
 (segment (start 35.08509 26.5675) (end 33.0425 26.5675) (width 0.2) (layer "F.Cu") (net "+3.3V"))
 (segment (start 54.757244 13.525) (end 55.0725 13.840256) (width 0.2) (layer "F.Cu") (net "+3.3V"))
 (segment (start 32.2425 27.0675) (end 33.0425 27.0675) (width 0.2) (layer "F.Cu") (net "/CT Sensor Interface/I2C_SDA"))
 (segment (start 40.00509 35.7875) (end 32.0175 27.79991) (width 0.2) (layer "F.Cu") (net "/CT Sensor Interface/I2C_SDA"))
 (segment (start 32.0175 27.2925) (end 32.2425 27.0675) (width 0.2) (layer "F.Cu") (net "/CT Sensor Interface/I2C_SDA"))
 (segment (start 32.0175 27.79991) (end 32.0175 27.2925) (width 0.2) (layer "F.Cu") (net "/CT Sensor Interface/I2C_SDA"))
 (segment (start 52.2925 35.7875) (end 40.00509 35.7875) (width 0.2) (layer "F.Cu") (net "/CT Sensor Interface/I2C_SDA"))
 (segment (start 38.7225 33.2475) (end 33.0425 27.5675) (width 0.2) (layer "F.Cu") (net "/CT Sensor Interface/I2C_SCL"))
 (segment (start 52.2925 33.2475) (end 38.7225 33.2475) (width 0.2) (layer "F.Cu") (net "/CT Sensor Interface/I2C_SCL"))
 (segment (start 16.58 24.64) (end 21.91 19.31) (width 0.2) (layer "F.Cu") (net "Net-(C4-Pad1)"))
 (segment (start 36.1025 16.2) (end 39.59 16.2) (width 0.2) (layer "F.Cu") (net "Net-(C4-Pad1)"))
 (segment (start 21.91 19.31) (end 33.39 19.31) (width 0.2) (layer "F.Cu") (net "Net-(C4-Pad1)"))
 (segment (start 45.1025 14.3375) (end 54.0725 14.3375) (width 0.2) (layer "F.Cu") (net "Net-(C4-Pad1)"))
 (segment (start 39.59 16.2) (end 41.4525 14.3375) (width 0.2) (layer "F.Cu") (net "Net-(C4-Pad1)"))
 (segment (start 41.4525 14.3375) (end 45.1025 14.3375) (width 0.2) (layer "F.Cu") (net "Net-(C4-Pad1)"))
 (segment (start 36.1025 16.5975) (end 36.1025 16.2) (width 0.2) (layer "F.Cu") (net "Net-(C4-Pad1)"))
 (segment (start 16.58 30.44) (end 16.58 24.64) (width 0.2) (layer "F.Cu") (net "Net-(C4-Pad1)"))
 (segment (start 33.39 19.31) (end 36.1025 16.5975) (width 0.2) (layer "F.Cu") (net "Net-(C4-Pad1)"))
 (segment (start 52.2925 30.7075) (end 53.4425 31.8575) (width 0.2) (layer "F.Cu") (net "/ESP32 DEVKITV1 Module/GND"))
 (segment (start 53.4425 37.1775) (end 52.2925 38.3275) (width 0.2) (layer "F.Cu") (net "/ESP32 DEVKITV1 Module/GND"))
 (segment (start 24.0775 38.3275) (end 24.01 38.26) (width 0.2) (layer "F.Cu") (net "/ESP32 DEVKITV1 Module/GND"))
 (segment (start 53.4425 31.8575) (end 53.4425 37.1775) (width 0.2) (layer "F.Cu") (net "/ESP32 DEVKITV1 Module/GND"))
 (segment (start 52.2925 38.3275) (end 24.0775 38.3275) (width 0.2) (layer "F.Cu") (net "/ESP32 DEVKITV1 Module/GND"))
 (segment (start 18.93 38.26) (end 14.1675 33.4975) (width 0.2) (layer "F.Cu") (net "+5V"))
 (segment (start 14.1675 16.8525) (end 17.0325 13.9875) (width 0.2) (layer "F.Cu") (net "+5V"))
 (segment (start 14.1675 33.4975) (end 14.1675 16.8525) (width 0.2) (layer "F.Cu") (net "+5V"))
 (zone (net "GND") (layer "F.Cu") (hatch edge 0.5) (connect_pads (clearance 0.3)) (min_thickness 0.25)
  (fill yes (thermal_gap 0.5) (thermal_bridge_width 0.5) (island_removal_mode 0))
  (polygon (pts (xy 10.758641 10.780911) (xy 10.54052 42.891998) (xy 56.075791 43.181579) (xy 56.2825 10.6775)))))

